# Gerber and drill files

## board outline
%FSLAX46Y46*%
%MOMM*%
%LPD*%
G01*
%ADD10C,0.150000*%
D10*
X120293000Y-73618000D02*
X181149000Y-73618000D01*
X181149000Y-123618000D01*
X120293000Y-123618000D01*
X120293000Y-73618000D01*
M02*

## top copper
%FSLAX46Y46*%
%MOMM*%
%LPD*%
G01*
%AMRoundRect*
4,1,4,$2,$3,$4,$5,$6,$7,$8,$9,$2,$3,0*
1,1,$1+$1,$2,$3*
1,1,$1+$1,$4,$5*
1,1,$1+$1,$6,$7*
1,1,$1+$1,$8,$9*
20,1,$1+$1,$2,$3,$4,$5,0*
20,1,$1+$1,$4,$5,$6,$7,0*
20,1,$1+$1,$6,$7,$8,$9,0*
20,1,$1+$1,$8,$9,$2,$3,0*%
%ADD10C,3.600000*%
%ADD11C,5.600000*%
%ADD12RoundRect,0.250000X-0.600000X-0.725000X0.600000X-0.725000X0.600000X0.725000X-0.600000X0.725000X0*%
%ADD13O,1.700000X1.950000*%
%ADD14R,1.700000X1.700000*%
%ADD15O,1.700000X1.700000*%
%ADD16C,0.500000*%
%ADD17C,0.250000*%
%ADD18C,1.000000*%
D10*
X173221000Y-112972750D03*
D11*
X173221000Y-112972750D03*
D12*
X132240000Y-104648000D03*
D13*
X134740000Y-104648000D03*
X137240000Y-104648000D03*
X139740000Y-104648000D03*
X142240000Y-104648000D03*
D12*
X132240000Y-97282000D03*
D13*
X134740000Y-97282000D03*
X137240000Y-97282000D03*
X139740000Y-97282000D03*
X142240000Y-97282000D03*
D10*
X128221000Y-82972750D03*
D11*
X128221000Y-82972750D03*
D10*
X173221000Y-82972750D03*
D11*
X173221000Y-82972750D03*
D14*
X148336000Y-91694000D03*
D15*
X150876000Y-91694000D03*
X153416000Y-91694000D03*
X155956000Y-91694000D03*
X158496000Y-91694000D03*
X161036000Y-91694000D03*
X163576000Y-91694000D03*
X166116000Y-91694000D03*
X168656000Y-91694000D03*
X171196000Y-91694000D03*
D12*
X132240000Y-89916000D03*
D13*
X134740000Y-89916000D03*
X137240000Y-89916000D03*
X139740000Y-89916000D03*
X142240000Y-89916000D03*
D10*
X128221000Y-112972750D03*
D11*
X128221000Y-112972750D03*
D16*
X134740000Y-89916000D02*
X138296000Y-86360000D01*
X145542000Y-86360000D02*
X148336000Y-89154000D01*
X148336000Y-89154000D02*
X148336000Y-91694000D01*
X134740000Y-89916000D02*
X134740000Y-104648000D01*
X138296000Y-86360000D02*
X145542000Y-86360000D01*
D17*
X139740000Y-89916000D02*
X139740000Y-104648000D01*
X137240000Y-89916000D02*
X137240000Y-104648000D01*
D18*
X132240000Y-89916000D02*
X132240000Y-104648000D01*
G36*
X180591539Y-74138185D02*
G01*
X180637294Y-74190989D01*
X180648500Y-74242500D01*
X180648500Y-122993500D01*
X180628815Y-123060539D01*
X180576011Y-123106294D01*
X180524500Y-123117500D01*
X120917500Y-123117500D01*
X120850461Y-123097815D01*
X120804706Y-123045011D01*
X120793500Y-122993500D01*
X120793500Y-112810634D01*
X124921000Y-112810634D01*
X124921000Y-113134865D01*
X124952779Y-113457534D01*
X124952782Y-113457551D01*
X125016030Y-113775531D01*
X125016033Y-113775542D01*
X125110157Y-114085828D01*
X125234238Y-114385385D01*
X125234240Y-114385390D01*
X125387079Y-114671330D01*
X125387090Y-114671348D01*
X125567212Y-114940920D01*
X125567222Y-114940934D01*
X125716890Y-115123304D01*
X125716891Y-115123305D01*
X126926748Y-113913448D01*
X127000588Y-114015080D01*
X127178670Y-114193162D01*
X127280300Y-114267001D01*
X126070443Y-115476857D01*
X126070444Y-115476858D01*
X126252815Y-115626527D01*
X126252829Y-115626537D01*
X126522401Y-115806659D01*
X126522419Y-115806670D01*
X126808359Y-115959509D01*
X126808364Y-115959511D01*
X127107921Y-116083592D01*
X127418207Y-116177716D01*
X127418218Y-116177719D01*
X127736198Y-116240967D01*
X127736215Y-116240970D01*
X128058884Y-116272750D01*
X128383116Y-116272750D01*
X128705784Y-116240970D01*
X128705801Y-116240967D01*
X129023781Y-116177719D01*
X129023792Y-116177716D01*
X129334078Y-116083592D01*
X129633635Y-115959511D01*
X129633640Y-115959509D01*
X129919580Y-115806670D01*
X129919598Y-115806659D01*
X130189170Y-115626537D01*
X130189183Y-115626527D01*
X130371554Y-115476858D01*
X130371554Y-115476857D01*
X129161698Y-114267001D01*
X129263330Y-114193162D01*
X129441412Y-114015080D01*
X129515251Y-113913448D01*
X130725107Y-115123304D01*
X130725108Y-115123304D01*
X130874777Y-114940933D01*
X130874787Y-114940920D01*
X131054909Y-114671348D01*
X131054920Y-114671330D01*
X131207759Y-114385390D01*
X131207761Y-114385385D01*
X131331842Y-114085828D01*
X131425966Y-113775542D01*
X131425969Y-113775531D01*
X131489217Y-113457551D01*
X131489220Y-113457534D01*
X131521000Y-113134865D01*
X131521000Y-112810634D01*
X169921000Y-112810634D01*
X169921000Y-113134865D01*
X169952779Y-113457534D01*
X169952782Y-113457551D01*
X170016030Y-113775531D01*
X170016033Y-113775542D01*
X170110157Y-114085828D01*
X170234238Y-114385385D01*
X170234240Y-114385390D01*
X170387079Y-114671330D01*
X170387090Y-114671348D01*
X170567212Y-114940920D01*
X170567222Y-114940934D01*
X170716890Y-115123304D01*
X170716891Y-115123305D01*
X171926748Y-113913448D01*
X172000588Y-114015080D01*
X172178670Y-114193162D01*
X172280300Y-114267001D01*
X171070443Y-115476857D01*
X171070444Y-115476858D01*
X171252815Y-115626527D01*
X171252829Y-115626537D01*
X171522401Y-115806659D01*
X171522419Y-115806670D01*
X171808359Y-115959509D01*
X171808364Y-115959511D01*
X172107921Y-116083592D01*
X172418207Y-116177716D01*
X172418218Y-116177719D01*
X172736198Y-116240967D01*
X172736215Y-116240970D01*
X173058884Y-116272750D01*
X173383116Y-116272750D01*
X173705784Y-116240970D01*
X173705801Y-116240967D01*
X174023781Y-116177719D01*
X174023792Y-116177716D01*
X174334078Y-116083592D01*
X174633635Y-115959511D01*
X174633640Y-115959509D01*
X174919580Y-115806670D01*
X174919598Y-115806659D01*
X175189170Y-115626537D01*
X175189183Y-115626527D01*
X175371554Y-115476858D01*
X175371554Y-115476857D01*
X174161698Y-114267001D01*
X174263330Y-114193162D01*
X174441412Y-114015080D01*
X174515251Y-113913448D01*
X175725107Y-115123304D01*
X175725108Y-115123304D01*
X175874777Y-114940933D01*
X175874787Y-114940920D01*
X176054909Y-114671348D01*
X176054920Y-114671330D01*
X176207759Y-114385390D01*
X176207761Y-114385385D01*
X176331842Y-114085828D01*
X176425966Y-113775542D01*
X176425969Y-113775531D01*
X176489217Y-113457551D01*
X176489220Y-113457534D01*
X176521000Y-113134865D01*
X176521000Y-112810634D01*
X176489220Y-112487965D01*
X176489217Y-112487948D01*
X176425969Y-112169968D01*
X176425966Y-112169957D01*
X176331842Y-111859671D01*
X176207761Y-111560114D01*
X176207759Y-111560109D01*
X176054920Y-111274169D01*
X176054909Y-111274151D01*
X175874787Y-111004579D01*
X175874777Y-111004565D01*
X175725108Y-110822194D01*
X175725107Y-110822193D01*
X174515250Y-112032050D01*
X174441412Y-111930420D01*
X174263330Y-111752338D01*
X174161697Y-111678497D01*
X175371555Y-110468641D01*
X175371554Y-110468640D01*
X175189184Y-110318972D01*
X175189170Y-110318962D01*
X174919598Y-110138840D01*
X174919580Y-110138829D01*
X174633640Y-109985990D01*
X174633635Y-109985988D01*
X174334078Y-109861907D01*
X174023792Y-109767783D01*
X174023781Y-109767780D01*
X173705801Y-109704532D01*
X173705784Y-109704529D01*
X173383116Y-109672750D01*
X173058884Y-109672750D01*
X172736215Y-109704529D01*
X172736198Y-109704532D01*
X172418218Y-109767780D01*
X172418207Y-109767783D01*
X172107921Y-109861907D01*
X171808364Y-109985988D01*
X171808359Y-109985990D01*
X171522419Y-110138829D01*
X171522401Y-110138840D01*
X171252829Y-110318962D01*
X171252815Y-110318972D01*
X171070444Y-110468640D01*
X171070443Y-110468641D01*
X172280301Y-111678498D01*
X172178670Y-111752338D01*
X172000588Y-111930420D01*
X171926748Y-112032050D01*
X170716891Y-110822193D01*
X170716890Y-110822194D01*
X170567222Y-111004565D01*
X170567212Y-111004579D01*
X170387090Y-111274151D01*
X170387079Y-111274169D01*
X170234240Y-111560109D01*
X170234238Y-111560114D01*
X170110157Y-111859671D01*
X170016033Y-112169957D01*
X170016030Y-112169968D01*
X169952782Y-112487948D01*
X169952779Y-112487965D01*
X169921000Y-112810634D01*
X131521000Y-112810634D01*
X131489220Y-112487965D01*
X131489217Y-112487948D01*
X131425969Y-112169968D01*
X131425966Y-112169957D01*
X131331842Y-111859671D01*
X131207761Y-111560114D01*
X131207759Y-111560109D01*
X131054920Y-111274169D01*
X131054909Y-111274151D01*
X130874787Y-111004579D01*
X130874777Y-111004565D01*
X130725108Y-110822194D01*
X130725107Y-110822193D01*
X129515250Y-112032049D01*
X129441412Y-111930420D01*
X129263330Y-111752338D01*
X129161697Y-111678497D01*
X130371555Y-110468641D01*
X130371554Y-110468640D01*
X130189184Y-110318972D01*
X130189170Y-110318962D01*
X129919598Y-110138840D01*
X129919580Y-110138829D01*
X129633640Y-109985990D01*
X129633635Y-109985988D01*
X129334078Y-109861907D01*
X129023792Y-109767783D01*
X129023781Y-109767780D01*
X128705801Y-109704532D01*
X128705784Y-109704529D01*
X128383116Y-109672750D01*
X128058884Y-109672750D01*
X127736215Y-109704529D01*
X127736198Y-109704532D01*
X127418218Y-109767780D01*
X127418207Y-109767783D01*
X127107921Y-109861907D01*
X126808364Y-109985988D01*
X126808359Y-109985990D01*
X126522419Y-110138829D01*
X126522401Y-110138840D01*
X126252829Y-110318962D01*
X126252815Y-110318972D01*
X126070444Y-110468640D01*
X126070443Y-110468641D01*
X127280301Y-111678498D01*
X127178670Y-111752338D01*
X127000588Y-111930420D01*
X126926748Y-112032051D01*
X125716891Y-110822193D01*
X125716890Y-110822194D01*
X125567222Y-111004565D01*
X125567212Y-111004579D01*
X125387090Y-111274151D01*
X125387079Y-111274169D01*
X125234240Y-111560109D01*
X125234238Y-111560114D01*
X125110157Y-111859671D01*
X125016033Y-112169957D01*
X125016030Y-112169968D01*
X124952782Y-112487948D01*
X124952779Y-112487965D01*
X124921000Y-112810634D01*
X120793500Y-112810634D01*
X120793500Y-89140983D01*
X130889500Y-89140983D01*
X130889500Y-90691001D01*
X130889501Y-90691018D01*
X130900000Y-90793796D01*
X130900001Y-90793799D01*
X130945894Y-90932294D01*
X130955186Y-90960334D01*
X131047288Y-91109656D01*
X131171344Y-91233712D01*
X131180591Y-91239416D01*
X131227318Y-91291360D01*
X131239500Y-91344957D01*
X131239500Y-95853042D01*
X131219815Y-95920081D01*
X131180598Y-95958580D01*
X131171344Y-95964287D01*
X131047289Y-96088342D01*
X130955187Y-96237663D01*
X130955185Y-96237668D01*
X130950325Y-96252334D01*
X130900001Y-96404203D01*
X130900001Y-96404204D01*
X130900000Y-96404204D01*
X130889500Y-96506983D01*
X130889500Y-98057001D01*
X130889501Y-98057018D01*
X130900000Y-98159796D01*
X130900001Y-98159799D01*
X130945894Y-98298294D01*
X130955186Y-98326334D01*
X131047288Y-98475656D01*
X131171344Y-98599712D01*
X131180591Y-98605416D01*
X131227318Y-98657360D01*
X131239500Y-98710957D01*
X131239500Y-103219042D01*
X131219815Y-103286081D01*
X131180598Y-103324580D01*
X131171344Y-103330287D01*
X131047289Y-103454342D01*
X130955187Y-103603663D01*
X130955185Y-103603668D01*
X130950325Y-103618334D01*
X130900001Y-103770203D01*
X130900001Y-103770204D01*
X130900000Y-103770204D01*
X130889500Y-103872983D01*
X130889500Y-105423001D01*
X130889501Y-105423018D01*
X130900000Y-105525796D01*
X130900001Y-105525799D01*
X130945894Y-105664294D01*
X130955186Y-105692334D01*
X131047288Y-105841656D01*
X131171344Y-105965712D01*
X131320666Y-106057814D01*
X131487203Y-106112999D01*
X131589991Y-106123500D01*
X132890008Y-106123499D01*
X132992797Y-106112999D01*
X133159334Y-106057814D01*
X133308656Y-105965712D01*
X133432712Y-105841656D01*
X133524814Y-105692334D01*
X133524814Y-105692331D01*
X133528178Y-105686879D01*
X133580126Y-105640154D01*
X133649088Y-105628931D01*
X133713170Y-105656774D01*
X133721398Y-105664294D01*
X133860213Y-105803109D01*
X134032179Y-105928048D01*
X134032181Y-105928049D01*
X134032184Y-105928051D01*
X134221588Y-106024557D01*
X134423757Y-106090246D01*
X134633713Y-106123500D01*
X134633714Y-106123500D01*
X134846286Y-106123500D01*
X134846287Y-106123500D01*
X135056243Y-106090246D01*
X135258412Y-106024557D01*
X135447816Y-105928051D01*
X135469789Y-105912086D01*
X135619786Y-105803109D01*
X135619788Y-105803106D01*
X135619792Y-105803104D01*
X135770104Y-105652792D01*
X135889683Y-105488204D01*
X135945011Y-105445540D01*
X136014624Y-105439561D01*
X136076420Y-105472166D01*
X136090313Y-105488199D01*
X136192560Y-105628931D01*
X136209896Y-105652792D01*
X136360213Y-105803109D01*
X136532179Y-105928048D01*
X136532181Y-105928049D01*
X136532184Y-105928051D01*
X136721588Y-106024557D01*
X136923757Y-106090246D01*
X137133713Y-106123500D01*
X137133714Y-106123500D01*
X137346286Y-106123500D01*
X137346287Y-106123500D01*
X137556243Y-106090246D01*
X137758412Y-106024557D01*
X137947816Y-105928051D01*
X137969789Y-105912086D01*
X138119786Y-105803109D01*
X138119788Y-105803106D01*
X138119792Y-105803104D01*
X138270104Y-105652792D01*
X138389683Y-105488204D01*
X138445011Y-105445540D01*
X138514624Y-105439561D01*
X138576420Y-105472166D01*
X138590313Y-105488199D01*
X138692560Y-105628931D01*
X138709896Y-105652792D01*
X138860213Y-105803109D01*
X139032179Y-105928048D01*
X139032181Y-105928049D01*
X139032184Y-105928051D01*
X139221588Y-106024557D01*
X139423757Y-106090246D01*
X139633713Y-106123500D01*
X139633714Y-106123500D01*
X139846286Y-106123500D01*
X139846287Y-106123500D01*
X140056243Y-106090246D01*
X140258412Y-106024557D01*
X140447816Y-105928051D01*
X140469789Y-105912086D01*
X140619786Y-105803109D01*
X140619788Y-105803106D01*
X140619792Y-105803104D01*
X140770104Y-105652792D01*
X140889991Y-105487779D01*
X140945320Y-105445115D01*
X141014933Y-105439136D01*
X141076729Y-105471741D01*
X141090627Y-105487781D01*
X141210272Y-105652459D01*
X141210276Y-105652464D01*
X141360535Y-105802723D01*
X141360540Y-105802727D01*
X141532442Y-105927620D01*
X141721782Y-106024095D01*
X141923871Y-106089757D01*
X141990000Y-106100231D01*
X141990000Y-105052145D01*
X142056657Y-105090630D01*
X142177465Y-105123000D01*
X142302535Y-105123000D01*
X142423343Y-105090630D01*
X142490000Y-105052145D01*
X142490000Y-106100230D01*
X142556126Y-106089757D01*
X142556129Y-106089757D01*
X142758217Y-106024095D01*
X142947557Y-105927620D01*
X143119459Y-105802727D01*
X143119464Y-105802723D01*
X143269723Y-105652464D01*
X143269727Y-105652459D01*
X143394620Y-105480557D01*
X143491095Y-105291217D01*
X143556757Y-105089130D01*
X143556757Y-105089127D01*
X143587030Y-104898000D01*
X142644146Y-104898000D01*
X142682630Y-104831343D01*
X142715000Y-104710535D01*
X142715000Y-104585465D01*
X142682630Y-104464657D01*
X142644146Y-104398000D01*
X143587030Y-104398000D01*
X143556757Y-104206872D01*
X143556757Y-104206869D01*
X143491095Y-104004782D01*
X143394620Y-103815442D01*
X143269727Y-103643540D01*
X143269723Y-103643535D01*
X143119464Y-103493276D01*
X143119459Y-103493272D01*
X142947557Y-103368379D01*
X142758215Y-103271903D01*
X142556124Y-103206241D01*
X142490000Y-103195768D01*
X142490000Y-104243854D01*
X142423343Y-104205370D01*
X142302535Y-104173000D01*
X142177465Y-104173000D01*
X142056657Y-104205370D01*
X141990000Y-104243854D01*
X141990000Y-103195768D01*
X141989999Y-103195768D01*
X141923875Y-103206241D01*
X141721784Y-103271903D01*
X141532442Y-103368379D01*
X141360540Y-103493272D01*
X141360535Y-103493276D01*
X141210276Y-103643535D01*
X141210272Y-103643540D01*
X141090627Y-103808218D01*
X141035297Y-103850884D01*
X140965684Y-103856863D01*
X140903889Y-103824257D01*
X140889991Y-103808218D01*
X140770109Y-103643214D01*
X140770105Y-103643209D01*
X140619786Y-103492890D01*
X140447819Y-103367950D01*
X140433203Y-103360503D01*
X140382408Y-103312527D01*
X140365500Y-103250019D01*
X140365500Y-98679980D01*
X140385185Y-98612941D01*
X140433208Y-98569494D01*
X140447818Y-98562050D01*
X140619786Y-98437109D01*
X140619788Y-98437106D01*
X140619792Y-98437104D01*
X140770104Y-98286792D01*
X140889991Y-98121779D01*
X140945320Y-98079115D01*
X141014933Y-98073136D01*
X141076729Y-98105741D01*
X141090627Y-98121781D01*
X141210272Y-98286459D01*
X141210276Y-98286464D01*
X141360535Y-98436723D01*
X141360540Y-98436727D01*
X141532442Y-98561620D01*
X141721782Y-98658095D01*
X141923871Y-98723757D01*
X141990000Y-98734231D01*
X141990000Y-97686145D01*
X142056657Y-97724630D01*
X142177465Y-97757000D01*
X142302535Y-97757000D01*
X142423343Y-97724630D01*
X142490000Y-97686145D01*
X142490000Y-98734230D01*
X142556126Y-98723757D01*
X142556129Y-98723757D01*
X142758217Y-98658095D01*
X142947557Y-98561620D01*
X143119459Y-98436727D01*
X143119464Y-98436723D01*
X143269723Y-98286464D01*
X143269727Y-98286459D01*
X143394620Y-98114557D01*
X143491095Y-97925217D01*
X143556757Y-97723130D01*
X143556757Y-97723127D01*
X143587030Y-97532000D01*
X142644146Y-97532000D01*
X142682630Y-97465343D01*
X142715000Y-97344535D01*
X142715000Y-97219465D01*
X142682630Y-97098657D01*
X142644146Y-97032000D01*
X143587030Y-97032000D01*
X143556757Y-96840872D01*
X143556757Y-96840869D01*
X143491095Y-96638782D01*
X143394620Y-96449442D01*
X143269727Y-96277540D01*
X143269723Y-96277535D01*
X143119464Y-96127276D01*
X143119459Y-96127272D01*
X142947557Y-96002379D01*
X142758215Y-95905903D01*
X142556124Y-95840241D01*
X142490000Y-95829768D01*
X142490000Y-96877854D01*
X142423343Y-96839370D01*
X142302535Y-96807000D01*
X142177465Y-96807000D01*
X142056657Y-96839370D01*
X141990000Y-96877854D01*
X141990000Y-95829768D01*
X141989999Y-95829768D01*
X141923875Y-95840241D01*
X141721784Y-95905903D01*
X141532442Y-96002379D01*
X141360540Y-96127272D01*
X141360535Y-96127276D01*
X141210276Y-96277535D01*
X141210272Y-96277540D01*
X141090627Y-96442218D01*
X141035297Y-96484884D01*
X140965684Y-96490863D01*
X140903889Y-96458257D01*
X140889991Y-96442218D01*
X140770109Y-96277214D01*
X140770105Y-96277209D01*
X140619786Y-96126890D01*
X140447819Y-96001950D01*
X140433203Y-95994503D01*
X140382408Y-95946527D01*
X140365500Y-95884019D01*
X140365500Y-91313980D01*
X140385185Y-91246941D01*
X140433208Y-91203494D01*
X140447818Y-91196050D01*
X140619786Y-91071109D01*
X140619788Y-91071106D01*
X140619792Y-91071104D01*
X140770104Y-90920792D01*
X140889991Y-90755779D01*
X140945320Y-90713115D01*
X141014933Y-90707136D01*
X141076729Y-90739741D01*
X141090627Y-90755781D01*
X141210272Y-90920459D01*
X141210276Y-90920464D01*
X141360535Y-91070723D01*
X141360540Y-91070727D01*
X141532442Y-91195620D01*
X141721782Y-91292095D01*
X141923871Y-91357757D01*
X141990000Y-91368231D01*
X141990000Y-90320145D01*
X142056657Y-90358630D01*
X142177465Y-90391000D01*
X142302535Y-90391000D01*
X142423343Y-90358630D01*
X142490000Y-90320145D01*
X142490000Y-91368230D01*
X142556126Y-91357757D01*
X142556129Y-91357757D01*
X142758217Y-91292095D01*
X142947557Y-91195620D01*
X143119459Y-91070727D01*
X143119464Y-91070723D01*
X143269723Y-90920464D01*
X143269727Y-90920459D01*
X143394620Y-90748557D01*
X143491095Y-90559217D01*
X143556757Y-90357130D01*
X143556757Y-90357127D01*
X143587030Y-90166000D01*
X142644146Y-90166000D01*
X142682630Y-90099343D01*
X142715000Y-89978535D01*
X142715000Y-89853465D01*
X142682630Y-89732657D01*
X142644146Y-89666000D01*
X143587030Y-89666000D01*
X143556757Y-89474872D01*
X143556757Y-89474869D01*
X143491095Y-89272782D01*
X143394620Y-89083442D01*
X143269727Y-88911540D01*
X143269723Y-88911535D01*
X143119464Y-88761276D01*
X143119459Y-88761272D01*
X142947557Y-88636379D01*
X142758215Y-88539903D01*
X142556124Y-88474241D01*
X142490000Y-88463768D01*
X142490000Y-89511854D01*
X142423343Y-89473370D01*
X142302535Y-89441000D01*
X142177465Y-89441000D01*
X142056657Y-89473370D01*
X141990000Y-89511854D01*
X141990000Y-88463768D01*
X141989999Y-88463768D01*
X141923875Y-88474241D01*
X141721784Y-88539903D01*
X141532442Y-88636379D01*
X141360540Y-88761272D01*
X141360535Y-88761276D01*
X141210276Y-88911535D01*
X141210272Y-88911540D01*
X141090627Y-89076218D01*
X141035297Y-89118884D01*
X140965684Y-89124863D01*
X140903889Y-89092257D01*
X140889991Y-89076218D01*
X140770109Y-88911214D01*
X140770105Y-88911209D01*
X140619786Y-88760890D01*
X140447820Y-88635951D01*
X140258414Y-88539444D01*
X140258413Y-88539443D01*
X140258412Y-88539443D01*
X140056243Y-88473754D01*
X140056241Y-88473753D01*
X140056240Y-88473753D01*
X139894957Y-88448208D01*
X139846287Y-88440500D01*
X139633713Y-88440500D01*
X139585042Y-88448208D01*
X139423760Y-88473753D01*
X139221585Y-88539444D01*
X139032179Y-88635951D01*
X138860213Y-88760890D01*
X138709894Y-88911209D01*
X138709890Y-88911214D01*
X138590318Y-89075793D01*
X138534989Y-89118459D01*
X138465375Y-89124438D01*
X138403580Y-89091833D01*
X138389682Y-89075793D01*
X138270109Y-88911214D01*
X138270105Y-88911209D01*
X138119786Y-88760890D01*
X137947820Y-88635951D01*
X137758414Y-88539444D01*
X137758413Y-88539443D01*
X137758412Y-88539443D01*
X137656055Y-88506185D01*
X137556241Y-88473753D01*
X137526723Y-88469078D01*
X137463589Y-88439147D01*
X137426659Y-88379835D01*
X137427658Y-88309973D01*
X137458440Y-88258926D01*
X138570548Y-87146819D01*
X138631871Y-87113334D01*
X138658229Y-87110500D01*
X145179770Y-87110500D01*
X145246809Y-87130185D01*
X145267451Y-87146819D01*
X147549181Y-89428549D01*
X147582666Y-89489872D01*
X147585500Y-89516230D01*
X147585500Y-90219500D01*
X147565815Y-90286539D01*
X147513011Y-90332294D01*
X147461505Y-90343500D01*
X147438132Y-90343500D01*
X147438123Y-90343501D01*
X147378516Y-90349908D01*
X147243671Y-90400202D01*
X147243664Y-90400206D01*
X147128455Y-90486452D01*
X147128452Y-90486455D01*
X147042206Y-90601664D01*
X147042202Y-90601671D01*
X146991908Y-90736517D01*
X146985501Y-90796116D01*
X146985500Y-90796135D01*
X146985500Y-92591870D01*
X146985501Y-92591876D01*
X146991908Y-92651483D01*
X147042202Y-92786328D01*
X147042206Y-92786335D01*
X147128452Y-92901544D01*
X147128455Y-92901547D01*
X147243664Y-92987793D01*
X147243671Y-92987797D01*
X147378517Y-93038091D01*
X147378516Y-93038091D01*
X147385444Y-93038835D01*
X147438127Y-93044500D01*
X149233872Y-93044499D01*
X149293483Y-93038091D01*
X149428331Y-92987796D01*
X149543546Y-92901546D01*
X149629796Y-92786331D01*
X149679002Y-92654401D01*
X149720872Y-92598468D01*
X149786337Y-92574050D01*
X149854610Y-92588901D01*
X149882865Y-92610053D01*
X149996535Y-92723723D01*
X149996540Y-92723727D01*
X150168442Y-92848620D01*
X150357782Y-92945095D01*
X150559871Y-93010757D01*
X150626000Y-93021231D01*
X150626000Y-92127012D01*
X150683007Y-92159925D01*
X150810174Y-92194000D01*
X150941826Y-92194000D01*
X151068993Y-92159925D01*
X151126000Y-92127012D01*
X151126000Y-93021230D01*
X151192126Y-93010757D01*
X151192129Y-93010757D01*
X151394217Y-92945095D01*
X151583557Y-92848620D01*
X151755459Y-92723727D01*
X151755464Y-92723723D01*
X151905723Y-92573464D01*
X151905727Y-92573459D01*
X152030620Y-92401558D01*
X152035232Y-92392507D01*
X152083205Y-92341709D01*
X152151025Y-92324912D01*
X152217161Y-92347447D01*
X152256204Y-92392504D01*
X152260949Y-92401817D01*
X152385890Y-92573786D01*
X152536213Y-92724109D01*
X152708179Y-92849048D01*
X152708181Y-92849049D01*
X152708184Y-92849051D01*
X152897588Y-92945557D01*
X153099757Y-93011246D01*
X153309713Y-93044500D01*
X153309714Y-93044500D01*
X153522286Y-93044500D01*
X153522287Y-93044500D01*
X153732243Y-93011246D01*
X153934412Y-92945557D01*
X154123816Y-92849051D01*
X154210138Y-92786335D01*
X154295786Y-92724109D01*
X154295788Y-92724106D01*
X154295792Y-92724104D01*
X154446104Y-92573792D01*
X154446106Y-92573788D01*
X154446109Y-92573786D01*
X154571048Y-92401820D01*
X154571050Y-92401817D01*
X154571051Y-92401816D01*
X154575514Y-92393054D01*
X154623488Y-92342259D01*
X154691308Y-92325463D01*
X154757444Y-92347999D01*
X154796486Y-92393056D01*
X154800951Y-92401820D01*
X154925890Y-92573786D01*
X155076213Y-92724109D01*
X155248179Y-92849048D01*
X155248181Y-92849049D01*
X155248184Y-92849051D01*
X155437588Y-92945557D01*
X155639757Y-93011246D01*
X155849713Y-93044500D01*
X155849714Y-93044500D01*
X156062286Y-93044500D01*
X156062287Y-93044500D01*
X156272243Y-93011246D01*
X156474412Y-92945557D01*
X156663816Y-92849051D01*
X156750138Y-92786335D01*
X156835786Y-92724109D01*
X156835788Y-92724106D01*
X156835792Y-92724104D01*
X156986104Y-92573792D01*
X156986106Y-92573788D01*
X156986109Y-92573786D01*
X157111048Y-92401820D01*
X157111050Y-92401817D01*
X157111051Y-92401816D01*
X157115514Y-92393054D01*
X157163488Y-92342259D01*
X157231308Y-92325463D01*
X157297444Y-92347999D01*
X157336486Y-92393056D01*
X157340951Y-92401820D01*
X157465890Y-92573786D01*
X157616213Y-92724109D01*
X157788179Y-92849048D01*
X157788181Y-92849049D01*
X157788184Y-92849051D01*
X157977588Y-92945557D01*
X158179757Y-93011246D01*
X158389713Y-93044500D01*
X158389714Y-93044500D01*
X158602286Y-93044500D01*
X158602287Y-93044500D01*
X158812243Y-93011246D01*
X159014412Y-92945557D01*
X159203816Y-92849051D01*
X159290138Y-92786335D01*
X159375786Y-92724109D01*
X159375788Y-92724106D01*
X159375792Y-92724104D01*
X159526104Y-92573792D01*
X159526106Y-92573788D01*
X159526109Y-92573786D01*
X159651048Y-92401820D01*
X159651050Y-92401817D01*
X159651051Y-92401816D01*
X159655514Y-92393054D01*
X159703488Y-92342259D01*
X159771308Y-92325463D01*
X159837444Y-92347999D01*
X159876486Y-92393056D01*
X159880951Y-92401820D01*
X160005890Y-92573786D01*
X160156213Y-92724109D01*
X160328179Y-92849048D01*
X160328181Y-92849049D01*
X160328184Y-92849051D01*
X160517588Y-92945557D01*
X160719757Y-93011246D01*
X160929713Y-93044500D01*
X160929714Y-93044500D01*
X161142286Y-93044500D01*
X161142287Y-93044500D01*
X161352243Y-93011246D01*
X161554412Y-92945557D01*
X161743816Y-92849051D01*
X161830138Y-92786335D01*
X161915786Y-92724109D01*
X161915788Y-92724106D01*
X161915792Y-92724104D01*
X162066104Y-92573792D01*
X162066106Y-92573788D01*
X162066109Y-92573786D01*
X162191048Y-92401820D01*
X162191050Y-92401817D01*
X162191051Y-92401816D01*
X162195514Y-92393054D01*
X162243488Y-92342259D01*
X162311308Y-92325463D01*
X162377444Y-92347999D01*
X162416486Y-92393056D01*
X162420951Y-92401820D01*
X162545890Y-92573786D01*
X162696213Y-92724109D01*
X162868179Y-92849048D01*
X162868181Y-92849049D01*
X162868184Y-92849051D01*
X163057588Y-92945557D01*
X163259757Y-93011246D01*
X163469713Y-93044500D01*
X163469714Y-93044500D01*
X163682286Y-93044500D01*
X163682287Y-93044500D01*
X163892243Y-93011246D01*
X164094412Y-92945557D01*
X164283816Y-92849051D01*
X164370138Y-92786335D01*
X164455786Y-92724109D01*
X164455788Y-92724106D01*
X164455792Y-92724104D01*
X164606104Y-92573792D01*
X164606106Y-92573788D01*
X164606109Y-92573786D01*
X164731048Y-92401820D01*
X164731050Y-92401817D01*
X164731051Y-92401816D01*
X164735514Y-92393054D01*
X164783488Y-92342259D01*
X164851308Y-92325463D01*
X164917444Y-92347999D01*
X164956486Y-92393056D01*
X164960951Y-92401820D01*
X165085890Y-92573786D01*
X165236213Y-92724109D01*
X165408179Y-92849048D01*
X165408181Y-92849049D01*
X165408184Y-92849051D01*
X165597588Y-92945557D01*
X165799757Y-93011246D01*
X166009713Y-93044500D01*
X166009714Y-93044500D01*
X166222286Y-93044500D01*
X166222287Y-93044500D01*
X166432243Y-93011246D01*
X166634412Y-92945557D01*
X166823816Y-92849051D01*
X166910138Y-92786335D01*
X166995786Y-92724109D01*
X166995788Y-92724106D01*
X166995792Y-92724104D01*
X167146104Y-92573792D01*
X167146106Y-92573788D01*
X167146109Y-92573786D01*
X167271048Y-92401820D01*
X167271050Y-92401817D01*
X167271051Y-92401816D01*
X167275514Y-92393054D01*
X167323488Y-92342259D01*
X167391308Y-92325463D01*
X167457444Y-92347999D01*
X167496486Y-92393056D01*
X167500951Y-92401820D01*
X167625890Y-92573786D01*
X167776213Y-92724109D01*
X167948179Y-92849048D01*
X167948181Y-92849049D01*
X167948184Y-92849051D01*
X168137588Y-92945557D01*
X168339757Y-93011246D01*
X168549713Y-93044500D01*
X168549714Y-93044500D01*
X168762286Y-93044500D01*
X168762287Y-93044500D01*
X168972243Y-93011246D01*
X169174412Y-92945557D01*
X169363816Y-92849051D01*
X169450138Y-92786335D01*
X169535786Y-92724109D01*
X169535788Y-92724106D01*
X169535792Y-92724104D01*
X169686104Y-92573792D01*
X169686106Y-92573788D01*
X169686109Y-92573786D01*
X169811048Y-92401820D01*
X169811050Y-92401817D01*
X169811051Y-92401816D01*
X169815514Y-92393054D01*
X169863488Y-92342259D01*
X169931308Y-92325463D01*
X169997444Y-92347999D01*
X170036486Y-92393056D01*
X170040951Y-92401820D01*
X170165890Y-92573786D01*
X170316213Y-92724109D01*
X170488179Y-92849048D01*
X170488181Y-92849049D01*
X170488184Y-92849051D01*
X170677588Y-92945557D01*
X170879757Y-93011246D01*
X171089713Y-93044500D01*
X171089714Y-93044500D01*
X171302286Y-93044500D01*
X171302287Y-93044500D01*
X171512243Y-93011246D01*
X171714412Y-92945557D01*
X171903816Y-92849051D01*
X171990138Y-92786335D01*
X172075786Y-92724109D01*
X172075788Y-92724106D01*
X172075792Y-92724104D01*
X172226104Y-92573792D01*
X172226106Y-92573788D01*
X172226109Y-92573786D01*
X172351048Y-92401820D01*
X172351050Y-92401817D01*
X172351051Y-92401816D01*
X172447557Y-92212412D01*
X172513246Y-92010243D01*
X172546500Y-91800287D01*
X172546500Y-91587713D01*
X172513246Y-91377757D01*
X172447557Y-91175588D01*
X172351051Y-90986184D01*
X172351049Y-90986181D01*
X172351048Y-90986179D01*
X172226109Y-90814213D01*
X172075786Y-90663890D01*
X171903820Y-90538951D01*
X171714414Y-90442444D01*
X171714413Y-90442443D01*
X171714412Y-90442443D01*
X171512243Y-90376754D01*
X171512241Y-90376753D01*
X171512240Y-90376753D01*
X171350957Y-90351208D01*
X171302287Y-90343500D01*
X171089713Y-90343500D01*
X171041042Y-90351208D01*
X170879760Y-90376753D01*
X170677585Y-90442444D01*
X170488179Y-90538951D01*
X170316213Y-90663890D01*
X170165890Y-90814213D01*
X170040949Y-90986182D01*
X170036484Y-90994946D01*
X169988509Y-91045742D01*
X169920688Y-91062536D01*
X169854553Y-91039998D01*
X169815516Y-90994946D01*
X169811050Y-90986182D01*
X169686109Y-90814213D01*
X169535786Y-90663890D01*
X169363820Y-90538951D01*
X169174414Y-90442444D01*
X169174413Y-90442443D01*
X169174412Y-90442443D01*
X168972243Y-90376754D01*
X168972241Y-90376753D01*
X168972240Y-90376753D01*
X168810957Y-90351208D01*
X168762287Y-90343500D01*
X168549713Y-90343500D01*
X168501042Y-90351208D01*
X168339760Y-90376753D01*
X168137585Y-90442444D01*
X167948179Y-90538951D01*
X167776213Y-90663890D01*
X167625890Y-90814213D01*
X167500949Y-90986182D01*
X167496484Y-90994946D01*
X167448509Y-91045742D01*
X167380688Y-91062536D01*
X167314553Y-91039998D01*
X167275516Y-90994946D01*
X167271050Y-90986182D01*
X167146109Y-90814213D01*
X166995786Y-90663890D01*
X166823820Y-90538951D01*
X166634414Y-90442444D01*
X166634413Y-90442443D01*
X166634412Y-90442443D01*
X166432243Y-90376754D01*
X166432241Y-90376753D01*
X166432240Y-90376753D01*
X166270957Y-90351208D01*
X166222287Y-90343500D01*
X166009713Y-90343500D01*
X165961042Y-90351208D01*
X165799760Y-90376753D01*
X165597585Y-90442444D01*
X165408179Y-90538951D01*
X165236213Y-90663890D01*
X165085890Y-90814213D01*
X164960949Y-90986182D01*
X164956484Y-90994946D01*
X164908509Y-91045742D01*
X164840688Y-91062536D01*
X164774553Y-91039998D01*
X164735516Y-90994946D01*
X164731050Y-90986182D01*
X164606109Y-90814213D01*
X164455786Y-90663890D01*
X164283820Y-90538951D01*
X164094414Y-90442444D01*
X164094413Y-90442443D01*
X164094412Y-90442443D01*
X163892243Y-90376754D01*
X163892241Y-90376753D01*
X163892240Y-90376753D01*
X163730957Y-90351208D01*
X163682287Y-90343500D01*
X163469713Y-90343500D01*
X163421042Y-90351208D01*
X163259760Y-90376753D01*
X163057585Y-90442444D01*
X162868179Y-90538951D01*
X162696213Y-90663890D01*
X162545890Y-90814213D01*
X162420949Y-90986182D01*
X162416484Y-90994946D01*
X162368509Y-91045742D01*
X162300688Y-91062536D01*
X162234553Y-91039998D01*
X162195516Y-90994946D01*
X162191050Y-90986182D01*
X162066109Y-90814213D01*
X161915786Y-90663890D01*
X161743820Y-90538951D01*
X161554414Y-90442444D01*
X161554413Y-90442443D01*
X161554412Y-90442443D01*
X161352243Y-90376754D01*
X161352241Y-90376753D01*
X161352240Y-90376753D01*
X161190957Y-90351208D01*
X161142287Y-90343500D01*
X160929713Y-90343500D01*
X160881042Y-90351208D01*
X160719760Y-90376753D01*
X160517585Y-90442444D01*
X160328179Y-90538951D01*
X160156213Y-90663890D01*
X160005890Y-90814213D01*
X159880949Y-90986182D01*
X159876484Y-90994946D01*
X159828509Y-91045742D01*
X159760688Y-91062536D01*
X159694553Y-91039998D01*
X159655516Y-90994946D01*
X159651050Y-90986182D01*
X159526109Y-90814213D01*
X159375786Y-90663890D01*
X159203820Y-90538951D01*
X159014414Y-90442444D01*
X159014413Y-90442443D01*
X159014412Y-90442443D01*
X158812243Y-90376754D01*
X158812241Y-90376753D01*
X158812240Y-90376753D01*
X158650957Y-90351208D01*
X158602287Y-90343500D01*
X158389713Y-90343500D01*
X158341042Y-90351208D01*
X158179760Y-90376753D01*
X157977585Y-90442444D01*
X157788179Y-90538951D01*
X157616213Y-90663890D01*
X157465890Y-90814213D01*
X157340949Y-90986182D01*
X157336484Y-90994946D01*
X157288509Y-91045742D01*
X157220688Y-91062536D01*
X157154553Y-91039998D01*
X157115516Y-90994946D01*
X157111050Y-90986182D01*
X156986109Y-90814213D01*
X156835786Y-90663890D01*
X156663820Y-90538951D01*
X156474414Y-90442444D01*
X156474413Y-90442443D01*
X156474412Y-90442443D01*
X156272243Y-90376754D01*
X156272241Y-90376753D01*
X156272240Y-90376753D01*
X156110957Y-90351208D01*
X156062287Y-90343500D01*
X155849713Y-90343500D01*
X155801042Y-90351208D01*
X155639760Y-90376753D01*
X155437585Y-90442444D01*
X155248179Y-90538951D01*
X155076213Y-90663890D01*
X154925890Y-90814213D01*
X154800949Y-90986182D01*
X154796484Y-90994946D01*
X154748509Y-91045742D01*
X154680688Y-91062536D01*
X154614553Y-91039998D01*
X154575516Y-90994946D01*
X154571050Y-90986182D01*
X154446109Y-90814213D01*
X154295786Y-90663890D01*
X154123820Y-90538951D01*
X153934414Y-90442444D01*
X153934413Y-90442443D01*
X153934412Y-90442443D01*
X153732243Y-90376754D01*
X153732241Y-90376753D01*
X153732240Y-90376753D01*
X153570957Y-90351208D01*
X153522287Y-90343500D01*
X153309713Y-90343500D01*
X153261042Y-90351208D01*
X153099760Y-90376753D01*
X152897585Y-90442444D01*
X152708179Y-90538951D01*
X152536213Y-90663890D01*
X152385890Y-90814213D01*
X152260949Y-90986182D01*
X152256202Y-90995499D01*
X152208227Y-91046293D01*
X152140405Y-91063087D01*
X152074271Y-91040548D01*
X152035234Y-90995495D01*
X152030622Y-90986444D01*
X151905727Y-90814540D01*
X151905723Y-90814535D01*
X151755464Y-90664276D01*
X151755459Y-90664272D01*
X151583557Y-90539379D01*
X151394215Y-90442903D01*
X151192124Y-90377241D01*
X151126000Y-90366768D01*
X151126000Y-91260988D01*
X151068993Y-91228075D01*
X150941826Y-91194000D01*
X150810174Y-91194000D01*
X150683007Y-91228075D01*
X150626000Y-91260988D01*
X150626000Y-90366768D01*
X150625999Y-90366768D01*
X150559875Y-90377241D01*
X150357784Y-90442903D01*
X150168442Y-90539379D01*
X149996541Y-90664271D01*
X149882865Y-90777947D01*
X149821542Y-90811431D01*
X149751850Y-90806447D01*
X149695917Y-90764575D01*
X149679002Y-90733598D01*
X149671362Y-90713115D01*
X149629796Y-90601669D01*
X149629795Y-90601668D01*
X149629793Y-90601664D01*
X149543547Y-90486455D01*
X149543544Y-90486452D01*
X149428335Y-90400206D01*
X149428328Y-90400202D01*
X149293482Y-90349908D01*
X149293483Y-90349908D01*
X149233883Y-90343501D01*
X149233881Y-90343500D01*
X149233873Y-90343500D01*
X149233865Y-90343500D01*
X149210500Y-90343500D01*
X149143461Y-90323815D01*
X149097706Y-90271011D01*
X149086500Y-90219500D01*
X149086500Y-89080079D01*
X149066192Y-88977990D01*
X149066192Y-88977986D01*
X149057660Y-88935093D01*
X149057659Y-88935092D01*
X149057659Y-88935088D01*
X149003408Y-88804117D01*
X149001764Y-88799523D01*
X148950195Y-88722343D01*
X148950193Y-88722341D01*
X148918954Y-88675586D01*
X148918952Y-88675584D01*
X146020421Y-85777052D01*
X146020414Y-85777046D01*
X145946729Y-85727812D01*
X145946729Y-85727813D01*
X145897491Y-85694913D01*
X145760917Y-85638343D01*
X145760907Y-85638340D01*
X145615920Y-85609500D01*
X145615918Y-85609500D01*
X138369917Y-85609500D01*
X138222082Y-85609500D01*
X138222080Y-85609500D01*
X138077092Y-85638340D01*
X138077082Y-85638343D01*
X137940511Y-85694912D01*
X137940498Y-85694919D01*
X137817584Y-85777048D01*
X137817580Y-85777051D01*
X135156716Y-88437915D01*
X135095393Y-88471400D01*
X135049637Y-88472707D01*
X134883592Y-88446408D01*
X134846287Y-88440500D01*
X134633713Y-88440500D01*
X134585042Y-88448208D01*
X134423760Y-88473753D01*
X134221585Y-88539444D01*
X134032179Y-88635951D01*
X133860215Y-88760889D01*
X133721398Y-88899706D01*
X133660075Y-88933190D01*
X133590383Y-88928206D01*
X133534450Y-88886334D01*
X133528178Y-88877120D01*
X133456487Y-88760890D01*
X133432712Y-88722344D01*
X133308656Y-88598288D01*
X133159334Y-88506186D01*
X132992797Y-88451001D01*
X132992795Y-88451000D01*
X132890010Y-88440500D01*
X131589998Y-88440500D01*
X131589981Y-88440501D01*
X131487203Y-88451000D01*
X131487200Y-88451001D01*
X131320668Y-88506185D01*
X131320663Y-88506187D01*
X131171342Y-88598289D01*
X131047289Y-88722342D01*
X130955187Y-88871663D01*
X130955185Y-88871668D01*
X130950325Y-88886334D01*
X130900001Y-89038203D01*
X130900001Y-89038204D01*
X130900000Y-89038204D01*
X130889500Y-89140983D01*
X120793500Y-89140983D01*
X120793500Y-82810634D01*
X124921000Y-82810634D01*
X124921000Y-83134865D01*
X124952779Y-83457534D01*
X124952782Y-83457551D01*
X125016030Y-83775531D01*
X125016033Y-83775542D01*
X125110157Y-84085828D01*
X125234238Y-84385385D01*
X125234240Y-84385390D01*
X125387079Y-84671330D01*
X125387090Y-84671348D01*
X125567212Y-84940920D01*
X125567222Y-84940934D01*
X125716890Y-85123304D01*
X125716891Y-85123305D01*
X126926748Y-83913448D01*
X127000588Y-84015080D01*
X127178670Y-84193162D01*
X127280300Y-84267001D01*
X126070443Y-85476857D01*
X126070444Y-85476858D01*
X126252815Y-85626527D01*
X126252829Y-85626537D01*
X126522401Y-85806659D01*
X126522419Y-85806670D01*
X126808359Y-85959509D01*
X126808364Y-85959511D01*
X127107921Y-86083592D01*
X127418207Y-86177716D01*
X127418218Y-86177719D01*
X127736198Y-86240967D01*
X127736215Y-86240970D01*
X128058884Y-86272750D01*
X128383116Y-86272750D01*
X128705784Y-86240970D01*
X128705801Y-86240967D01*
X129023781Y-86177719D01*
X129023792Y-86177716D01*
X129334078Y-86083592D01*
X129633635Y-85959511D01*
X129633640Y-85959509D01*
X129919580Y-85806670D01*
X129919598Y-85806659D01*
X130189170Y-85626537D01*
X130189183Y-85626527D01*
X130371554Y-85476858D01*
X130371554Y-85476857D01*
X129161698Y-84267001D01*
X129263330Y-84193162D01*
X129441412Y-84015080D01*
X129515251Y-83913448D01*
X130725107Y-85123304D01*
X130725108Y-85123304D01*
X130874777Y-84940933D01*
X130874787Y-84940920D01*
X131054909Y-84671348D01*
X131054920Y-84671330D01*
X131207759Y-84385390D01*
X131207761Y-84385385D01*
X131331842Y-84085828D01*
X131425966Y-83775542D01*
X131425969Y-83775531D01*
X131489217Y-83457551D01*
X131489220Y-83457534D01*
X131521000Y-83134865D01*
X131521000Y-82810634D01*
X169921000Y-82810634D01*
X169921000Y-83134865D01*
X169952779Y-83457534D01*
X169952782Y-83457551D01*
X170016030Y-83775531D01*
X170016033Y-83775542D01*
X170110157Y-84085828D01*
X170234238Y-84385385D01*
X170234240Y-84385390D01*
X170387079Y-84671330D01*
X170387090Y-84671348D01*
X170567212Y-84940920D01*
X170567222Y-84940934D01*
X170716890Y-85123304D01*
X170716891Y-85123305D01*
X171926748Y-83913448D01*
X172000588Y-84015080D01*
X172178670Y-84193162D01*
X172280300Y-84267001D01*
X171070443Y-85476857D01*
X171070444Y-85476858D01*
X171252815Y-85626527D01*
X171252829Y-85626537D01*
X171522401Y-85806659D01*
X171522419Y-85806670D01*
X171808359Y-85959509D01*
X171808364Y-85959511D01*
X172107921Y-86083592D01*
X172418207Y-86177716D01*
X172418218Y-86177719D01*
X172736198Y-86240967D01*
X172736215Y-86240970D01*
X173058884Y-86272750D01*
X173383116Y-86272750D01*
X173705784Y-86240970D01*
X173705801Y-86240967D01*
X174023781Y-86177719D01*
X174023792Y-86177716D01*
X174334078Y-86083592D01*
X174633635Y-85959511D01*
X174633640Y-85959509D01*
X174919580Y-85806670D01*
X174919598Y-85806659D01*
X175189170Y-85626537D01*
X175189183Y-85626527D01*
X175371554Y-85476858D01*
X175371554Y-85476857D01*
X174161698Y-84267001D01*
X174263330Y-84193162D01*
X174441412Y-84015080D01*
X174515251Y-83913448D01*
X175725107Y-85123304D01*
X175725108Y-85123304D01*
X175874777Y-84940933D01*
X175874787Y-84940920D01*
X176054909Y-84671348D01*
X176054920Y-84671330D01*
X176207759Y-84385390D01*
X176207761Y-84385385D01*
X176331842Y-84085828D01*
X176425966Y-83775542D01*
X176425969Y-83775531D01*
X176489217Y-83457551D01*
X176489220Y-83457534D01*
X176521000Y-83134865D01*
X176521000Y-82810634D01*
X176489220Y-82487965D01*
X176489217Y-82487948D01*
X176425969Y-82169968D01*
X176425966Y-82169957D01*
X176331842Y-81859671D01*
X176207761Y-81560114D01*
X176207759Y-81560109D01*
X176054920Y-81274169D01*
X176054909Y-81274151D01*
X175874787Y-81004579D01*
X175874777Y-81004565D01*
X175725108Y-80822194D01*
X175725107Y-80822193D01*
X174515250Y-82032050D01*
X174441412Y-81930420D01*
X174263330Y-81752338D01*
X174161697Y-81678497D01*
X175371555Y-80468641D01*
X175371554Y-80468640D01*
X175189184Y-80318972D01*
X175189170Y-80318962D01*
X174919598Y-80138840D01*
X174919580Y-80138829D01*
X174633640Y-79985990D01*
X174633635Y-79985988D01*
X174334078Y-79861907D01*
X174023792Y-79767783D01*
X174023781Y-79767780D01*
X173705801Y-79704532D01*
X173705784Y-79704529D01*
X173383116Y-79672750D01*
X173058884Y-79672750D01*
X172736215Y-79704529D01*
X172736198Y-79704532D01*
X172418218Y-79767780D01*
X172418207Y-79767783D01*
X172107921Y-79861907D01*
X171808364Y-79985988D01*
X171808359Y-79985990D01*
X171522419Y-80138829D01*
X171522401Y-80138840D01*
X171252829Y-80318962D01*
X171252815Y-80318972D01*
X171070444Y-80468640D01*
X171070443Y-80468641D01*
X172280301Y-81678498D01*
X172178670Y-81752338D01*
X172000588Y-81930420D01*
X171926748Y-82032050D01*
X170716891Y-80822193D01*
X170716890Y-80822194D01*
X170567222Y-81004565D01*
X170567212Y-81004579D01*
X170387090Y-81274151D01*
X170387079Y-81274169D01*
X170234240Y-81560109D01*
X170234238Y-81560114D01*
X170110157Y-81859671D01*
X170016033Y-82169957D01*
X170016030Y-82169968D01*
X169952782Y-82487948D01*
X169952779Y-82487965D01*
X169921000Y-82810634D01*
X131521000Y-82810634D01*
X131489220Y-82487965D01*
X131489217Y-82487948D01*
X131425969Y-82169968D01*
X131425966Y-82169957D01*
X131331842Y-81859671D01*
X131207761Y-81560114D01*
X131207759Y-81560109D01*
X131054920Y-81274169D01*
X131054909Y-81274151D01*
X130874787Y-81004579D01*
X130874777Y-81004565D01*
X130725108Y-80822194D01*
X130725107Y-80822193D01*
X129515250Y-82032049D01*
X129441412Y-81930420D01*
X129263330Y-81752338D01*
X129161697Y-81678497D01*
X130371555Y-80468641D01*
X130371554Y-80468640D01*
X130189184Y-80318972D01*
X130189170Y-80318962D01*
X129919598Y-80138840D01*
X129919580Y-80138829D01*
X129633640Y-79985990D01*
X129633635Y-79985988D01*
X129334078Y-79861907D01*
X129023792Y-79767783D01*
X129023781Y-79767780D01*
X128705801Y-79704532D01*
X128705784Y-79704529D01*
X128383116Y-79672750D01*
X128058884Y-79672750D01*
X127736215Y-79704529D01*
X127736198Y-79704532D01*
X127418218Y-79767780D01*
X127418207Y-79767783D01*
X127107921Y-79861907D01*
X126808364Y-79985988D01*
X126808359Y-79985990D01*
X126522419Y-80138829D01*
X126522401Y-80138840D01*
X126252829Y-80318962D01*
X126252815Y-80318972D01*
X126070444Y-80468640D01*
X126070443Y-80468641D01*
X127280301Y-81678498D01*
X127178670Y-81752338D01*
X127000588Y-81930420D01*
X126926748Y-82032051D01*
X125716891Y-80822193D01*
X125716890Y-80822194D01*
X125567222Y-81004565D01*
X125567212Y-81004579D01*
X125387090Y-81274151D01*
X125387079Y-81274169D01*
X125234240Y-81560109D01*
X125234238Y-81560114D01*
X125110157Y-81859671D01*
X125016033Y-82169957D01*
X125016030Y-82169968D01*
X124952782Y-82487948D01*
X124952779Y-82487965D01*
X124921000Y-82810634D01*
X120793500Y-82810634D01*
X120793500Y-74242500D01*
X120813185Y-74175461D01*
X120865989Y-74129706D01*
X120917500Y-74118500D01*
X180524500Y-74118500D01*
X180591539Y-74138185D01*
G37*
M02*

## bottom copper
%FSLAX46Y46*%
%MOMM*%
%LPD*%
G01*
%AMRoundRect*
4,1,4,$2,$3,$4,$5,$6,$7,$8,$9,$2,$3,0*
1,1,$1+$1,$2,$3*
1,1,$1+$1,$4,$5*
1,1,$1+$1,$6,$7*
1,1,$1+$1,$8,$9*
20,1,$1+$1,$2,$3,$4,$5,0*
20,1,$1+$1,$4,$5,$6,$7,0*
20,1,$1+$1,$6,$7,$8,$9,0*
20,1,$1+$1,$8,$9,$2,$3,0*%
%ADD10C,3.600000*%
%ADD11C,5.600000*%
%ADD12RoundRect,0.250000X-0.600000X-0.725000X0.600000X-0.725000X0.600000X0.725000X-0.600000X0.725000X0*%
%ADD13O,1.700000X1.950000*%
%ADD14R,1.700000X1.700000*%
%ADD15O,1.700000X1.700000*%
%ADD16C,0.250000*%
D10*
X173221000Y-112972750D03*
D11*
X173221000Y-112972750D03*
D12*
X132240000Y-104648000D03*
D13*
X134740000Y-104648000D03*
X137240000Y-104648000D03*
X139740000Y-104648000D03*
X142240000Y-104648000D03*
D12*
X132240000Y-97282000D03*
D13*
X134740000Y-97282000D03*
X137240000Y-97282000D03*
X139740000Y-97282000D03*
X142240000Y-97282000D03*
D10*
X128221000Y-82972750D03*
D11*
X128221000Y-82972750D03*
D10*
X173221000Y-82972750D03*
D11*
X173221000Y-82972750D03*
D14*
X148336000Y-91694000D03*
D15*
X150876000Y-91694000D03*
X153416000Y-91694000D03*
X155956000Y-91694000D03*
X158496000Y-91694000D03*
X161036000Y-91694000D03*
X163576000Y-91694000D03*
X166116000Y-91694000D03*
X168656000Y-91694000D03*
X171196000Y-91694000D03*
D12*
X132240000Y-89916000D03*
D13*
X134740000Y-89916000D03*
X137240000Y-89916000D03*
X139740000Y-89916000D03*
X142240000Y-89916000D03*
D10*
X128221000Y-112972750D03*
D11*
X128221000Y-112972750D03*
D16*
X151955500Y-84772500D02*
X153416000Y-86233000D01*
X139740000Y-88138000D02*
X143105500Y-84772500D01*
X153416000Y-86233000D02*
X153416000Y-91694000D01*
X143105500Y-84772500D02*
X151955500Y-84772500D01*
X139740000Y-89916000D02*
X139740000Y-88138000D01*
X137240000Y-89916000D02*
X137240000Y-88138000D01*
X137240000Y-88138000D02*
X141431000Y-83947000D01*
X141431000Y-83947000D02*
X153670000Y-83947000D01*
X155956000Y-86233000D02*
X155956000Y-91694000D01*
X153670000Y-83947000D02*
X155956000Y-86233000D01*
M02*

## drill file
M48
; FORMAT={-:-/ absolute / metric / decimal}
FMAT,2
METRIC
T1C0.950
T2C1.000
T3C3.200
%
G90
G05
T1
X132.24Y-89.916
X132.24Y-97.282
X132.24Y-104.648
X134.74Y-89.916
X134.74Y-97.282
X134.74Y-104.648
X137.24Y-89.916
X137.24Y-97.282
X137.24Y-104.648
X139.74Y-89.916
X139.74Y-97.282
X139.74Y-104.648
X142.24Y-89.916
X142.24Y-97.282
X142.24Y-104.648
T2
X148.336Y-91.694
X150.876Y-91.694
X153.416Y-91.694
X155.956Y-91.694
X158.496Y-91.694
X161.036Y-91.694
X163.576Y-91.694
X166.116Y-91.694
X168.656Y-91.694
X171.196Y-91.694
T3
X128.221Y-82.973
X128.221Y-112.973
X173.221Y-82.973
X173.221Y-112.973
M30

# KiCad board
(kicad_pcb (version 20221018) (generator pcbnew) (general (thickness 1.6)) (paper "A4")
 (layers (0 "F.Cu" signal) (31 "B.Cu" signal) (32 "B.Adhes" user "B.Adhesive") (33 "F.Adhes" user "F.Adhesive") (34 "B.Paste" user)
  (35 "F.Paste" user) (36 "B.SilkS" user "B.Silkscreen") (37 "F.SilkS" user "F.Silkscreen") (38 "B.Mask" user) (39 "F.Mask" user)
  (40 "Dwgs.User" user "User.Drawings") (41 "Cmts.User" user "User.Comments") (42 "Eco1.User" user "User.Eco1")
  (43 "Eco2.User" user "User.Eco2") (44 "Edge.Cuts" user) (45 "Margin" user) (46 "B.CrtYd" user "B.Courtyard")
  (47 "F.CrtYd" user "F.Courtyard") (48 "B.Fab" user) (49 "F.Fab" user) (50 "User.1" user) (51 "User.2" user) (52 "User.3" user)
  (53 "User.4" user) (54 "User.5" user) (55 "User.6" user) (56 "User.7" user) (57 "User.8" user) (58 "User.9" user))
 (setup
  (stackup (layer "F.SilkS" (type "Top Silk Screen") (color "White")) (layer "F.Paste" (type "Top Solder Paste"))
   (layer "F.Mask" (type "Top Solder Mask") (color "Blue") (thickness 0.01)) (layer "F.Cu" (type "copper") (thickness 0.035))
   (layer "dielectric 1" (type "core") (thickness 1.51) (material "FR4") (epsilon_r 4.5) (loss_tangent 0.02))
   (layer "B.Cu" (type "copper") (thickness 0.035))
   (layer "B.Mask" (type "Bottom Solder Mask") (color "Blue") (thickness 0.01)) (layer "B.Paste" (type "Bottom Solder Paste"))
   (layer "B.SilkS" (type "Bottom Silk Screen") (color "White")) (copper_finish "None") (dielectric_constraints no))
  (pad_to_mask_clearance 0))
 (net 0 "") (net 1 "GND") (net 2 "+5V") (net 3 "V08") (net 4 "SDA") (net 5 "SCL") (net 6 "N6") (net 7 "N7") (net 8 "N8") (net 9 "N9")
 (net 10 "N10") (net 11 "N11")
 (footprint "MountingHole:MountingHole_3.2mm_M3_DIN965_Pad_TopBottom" (layer "F.Cu") (at 173.221 112.97275)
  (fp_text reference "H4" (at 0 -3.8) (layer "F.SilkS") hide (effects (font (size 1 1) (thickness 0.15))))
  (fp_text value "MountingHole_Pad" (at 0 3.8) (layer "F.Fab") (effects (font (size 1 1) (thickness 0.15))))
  (pad "1" thru_hole circle (at 0 0) (size 3.6 3.6) (drill 3.2) (layers "*.Cu" "*.Mask") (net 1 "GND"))
  (pad "1" connect circle (at 0 0) (size 5.6 5.6) (layers "F.Cu" "F.Mask") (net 1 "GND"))
  (pad "1" connect circle (at 0 0) (size 5.6 5.6) (layers "B.Cu" "B.Mask") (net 1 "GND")))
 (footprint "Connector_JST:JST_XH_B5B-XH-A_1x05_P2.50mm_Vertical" (layer "F.Cu") (at 132.24 104.648)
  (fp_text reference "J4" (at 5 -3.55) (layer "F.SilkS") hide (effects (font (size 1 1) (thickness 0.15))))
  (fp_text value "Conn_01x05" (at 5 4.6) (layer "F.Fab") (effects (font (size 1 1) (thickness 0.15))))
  (pad "1" thru_hole roundrect (at 0 0) (size 1.7 1.95) (drill 0.95) (layers "*.Cu" "*.Mask") (roundrect_rratio 0.147059) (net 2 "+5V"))
  (pad "2" thru_hole oval (at 2.5 0) (size 1.7 1.95) (drill 0.95) (layers "*.Cu" "*.Mask") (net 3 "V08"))
  (pad "3" thru_hole oval (at 5 0) (size 1.7 1.95) (drill 0.95) (layers "*.Cu" "*.Mask") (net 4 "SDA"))
  (pad "4" thru_hole oval (at 7.5 0) (size 1.7 1.95) (drill 0.95) (layers "*.Cu" "*.Mask") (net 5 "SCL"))
  (pad "5" thru_hole oval (at 10 0) (size 1.7 1.95) (drill 0.95) (layers "*.Cu" "*.Mask") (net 1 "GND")))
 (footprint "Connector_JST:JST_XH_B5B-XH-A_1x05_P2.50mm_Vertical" (layer "F.Cu") (at 132.24 97.282)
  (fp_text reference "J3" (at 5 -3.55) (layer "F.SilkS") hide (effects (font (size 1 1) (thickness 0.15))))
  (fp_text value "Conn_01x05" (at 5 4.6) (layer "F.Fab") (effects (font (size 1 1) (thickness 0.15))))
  (pad "1" thru_hole roundrect (at 0 0) (size 1.7 1.95) (drill 0.95) (layers "*.Cu" "*.Mask") (roundrect_rratio 0.147059) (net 2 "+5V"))
  (pad "2" thru_hole oval (at 2.5 0) (size 1.7 1.95) (drill 0.95) (layers "*.Cu" "*.Mask") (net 3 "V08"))
  (pad "3" thru_hole oval (at 5 0) (size 1.7 1.95) (drill 0.95) (layers "*.Cu" "*.Mask") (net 4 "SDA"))
  (pad "4" thru_hole oval (at 7.5 0) (size 1.7 1.95) (drill 0.95) (layers "*.Cu" "*.Mask") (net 5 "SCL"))
  (pad "5" thru_hole oval (at 10 0) (size 1.7 1.95) (drill 0.95) (layers "*.Cu" "*.Mask") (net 1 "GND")))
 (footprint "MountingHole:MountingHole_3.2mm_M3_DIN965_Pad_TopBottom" (layer "F.Cu") (at 128.221 82.97275)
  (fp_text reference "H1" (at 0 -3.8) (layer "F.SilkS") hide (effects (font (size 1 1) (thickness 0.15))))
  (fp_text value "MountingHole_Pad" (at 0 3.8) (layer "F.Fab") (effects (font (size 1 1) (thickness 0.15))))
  (pad "1" thru_hole circle (at 0 0) (size 3.6 3.6) (drill 3.2) (layers "*.Cu" "*.Mask") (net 1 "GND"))
  (pad "1" connect circle (at 0 0) (size 5.6 5.6) (layers "F.Cu" "F.Mask") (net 1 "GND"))
  (pad "1" connect circle (at 0 0) (size 5.6 5.6) (layers "B.Cu" "B.Mask") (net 1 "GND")))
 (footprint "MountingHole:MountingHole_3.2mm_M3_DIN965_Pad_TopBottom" (layer "F.Cu") (at 173.221 82.97275)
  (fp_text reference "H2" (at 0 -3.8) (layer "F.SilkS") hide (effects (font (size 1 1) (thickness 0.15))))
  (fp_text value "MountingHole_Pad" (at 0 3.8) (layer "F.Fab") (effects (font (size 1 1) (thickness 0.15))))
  (pad "1" thru_hole circle (at 0 0) (size 3.6 3.6) (drill 3.2) (layers "*.Cu" "*.Mask") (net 1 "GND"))
  (pad "1" connect circle (at 0 0) (size 5.6 5.6) (layers "F.Cu" "F.Mask") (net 1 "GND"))
  (pad "1" connect circle (at 0 0) (size 5.6 5.6) (layers "B.Cu" "B.Mask") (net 1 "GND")))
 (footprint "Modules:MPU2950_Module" (layer "F.Cu") (at 159.766 80.264)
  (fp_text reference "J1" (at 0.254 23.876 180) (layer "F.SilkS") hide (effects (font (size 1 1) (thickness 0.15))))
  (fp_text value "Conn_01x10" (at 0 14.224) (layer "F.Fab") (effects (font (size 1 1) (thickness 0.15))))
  (pad "1" thru_hole rect (at -11.43 11.43 90) (size 1.7 1.7) (drill 1) (layers "*.Cu" "*.Mask") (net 3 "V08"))
  (pad "2" thru_hole oval (at -8.89 11.43 90) (size 1.7 1.7) (drill 1) (layers "*.Cu" "*.Mask") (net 1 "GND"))
  (pad "3" thru_hole oval (at -6.35 11.43 90) (size 1.7 1.7) (drill 1) (layers "*.Cu" "*.Mask") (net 5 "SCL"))
  (pad "4" thru_hole oval (at -3.81 11.43 90) (size 1.7 1.7) (drill 1) (layers "*.Cu" "*.Mask") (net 4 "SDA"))
  (pad "5" thru_hole oval (at -1.27 11.43 90) (size 1.7 1.7) (drill 1) (layers "*.Cu" "*.Mask") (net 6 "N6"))
  (pad "6" thru_hole oval (at 1.27 11.43 90) (size 1.7 1.7) (drill 1) (layers "*.Cu" "*.Mask") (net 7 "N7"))
  (pad "7" thru_hole oval (at 3.81 11.43 90) (size 1.7 1.7) (drill 1) (layers "*.Cu" "*.Mask") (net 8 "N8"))
  (pad "8" thru_hole oval (at 6.35 11.43 90) (size 1.7 1.7) (drill 1) (layers "*.Cu" "*.Mask") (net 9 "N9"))
  (pad "9" thru_hole oval (at 8.89 11.43 90) (size 1.7 1.7) (drill 1) (layers "*.Cu" "*.Mask") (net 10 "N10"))
  (pad "10" thru_hole oval (at 11.43 11.43 90) (size 1.7 1.7) (drill 1) (layers "*.Cu" "*.Mask") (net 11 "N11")))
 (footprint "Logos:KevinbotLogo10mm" (layer "F.Cu") (at 140.462 116.546)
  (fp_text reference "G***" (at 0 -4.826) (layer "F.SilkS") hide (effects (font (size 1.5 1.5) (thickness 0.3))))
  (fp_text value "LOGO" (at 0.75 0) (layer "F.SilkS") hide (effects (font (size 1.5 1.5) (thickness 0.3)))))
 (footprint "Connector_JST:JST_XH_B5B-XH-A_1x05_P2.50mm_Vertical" (layer "F.Cu") (at 132.24 89.916)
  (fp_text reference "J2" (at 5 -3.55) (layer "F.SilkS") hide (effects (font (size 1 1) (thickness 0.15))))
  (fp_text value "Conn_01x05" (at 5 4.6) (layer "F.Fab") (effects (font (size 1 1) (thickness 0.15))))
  (pad "1" thru_hole roundrect (at 0 0) (size 1.7 1.95) (drill 0.95) (layers "*.Cu" "*.Mask") (roundrect_rratio 0.147059) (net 2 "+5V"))
  (pad "2" thru_hole oval (at 2.5 0) (size 1.7 1.95) (drill 0.95) (layers "*.Cu" "*.Mask") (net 3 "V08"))
  (pad "3" thru_hole oval (at 5 0) (size 1.7 1.95) (drill 0.95) (layers "*.Cu" "*.Mask") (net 4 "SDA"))
  (pad "4" thru_hole oval (at 7.5 0) (size 1.7 1.95) (drill 0.95) (layers "*.Cu" "*.Mask") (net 5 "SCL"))
  (pad "5" thru_hole oval (at 10 0) (size 1.7 1.95) (drill 0.95) (layers "*.Cu" "*.Mask") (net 1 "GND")))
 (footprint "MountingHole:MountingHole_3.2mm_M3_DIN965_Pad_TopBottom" (layer "F.Cu") (at 128.221 112.97275)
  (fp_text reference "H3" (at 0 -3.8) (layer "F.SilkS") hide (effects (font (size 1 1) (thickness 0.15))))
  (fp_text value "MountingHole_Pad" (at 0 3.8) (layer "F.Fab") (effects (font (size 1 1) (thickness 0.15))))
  (pad "1" thru_hole circle (at 0 0) (size 3.6 3.6) (drill 3.2) (layers "*.Cu" "*.Mask") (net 1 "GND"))
  (pad "1" connect circle (at 0 0) (size 5.6 5.6) (layers "F.Cu" "F.Mask") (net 1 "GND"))
  (pad "1" connect circle (at 0 0) (size 5.6 5.6) (layers "B.Cu" "B.Mask") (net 1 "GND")))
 (gr_rect (start 120.293 73.618) (end 181.149 123.618) (stroke (width 0.15) (type default)) (fill none) (layer "Edge.Cuts"))
 (segment (start 134.74 89.916) (end 138.296 86.36) (width 0.5) (layer "F.Cu") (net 3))
 (segment (start 145.542 86.36) (end 148.336 89.154) (width 0.5) (layer "F.Cu") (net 3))
 (segment (start 148.336 89.154) (end 148.336 91.694) (width 0.5) (layer "F.Cu") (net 3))
 (segment (start 134.74 89.916) (end 134.74 104.648) (width 0.5) (layer "F.Cu") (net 3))
 (segment (start 138.296 86.36) (end 145.542 86.36) (width 0.5) (layer "F.Cu") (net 3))
 (segment (start 139.74 89.916) (end 139.74 104.648) (width 0.25) (layer "F.Cu") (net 5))
 (segment (start 151.9555 84.7725) (end 153.416 86.233) (width 0.25) (layer "B.Cu") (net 5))
 (segment (start 139.74 88.138) (end 143.1055 84.7725) (width 0.25) (layer "B.Cu") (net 5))
 (segment (start 153.416 86.233) (end 153.416 91.694) (width 0.25) (layer "B.Cu") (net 5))
 (segment (start 143.1055 84.7725) (end 151.9555 84.7725) (width 0.25) (layer "B.Cu") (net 5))
 (segment (start 139.74 89.916) (end 139.74 88.138) (width 0.25) (layer "B.Cu") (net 5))
 (segment (start 137.24 89.916) (end 137.24 104.648) (width 0.25) (layer "F.Cu") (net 4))
 (segment (start 137.24 89.916) (end 137.24 88.138) (width 0.25) (layer "B.Cu") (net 4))
 (segment (start 137.24 88.138) (end 141.431 83.947) (width 0.25) (layer "B.Cu") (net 4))
 (segment (start 141.431 83.947) (end 153.67 83.947) (width 0.25) (layer "B.Cu") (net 4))
 (segment (start 155.956 86.233) (end 155.956 91.694) (width 0.25) (layer "B.Cu") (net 4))
 (segment (start 153.67 83.947) (end 155.956 86.233) (width 0.25) (layer "B.Cu") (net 4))
 (segment (start 132.24 89.916) (end 132.24 104.648) (width 1) (layer "F.Cu") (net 2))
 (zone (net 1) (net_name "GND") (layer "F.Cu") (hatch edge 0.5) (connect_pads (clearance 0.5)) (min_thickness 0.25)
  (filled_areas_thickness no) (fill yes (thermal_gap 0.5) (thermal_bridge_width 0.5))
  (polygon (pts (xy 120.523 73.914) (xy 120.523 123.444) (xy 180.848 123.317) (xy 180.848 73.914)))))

